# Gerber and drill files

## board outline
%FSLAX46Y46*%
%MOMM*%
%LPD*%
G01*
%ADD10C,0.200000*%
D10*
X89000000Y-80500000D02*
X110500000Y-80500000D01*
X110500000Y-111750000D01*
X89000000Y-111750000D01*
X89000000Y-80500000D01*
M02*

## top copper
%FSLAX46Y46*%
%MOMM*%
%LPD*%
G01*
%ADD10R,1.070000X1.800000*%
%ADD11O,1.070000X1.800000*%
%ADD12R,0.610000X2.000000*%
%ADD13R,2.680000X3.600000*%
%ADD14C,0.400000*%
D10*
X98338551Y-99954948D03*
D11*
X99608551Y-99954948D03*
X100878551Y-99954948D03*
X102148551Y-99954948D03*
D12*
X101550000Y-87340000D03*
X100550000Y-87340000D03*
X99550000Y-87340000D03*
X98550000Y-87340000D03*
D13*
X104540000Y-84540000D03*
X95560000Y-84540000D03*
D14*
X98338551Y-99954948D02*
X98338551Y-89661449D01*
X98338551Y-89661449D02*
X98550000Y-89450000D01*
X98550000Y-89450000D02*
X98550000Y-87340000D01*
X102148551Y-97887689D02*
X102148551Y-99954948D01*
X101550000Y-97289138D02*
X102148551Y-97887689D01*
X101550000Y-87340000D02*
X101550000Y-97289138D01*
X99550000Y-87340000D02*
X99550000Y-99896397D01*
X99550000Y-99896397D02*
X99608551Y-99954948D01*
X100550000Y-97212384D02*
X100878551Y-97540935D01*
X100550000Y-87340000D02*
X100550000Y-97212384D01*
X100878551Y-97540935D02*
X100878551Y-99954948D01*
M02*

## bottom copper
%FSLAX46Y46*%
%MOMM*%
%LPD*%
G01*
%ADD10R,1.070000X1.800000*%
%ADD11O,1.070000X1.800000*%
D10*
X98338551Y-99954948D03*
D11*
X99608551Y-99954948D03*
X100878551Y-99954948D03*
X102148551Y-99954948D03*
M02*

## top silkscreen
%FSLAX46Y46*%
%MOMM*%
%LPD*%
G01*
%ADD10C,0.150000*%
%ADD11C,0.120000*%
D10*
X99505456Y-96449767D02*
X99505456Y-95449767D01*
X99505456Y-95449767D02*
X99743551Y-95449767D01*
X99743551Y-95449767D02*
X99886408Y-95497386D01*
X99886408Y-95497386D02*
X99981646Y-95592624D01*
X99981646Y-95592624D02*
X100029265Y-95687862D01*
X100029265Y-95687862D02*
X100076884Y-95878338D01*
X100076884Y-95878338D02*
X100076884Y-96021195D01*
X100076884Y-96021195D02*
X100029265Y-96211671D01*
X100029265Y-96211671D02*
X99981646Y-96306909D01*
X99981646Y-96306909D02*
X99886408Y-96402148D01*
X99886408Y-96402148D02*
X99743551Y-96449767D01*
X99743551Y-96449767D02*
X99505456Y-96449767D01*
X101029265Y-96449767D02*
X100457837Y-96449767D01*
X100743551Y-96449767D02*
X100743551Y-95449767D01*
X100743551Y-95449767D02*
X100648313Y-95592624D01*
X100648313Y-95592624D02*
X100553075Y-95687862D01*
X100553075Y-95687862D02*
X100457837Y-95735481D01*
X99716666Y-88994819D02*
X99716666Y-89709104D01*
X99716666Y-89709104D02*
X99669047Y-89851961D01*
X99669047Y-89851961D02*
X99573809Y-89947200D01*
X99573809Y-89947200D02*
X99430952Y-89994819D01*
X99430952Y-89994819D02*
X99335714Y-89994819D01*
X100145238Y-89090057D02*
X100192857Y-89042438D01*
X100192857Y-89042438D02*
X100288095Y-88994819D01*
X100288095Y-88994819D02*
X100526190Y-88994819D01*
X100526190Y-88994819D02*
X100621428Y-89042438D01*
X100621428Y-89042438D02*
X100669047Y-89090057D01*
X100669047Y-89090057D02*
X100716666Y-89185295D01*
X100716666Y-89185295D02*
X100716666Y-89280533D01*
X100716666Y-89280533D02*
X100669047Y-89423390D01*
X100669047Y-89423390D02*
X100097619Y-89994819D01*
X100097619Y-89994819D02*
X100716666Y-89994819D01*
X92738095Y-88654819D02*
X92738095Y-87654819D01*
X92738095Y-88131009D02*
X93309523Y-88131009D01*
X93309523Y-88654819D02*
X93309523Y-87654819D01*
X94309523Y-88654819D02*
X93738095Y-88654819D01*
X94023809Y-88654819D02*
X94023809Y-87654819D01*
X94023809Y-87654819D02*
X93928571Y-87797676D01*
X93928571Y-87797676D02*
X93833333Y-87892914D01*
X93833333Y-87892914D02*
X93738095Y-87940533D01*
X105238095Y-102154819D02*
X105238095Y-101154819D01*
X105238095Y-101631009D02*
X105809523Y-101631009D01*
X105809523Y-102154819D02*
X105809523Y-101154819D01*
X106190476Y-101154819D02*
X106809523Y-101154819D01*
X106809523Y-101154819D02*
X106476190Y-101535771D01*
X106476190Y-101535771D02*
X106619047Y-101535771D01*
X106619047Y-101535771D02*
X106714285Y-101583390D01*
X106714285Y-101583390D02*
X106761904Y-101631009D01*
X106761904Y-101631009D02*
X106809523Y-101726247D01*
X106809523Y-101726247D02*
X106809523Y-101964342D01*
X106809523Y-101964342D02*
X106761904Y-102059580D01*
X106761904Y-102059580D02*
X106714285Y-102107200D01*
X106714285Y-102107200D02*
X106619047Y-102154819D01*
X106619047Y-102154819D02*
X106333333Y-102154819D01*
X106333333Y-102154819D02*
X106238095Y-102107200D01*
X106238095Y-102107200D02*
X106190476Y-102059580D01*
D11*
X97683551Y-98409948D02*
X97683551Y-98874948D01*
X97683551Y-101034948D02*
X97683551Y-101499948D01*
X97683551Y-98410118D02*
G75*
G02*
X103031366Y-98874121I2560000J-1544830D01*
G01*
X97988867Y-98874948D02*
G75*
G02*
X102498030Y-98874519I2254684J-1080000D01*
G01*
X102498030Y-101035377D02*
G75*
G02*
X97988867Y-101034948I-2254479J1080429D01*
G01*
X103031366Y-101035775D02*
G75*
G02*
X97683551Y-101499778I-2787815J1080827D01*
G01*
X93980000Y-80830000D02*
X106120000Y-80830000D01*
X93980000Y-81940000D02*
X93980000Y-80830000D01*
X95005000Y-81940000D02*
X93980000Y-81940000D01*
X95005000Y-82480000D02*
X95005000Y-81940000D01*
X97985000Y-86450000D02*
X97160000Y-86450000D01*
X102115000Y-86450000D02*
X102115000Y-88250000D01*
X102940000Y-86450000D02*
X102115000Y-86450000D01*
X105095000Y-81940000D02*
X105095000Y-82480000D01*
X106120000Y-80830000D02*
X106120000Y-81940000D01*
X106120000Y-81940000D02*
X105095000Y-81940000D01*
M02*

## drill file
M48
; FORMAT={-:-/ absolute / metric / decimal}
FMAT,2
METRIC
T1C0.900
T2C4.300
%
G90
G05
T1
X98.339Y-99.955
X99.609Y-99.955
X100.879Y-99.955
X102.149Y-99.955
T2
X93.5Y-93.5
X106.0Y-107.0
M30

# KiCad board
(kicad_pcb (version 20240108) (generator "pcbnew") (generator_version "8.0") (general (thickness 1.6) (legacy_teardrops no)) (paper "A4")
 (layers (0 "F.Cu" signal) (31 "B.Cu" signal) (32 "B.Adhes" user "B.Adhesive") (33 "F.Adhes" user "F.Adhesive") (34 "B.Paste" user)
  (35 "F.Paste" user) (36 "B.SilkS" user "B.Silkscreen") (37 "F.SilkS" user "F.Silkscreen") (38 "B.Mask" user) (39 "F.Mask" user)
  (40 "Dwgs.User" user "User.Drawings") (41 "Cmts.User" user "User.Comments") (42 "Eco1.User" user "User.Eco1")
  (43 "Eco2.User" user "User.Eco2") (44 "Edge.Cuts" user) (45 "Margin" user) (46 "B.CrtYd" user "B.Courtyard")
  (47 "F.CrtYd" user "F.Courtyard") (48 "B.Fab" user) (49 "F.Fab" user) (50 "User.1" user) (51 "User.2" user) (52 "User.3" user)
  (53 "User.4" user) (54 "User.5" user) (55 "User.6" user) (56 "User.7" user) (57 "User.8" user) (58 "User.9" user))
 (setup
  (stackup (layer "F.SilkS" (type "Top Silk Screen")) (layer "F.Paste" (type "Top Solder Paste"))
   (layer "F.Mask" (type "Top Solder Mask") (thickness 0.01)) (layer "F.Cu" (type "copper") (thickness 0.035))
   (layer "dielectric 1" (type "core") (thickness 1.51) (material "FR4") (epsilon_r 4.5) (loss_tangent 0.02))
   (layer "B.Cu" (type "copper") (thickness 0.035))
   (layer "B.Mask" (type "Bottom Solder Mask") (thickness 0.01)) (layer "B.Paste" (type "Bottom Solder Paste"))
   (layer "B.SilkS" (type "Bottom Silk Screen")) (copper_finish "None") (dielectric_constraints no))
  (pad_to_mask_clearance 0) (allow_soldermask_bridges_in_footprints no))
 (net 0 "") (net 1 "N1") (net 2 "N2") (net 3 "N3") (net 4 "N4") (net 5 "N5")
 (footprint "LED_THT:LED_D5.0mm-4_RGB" (layer "F.Cu") (at 98.338551 99.954948)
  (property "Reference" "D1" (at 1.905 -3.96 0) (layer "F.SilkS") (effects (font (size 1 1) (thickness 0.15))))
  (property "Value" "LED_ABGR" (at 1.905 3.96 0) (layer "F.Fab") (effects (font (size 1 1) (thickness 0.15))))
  (fp_line (start -0.655 -1.545) (end -0.655 -1.08) (stroke (width 0.12) (type solid)) (layer "F.SilkS"))
  (fp_line (start -0.655 1.08) (end -0.655 1.545) (stroke (width 0.12) (type solid)) (layer "F.SilkS"))
  (fp_arc (start -0.655 -1.54483) (mid 2.163456 -2.978809) (end 4.692815 -1.080827) (stroke (width 0.12) (type solid)) (layer "F.SilkS"))
  (fp_arc (start -0.349684 -1.08) (mid 1.904762 -2.5) (end 4.159479 -1.080429) (stroke (width 0.12) (type solid)) (layer "F.SilkS"))
  (fp_arc (start 4.159479 1.080429) (mid 1.904762 2.5) (end -0.349684 1.08) (stroke (width 0.12) (type solid)) (layer "F.SilkS"))
  (fp_arc (start 4.692815 1.080827) (mid 2.163456 2.978808) (end -0.655 1.54483) (stroke (width 0.12) (type solid)) (layer "F.SilkS"))
  (pad "1" thru_hole rect (at 0 0) (size 1.07 1.8) (drill 0.9) (layers "*.Cu" "*.Mask") (remove_unused_layers no) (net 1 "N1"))
  (pad "2" thru_hole oval (at 1.27 0) (size 1.07 1.8) (drill 0.9) (layers "*.Cu" "*.Mask") (remove_unused_layers no) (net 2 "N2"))
  (pad "3" thru_hole oval (at 2.54 0) (size 1.07 1.8) (drill 0.9) (layers "*.Cu" "*.Mask") (remove_unused_layers no) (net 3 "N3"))
  (pad "4" thru_hole oval (at 3.81 0) (size 1.07 1.8) (drill 0.9) (layers "*.Cu" "*.Mask") (remove_unused_layers no) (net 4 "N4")))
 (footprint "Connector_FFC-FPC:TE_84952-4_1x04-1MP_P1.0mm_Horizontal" (layer "F.Cu") (at 100.05 85.54 180)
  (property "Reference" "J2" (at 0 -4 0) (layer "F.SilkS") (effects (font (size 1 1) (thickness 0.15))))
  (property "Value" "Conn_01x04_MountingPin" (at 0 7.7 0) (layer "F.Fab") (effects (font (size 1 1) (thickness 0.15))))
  (fp_line (start 6.07 4.71) (end -6.07 4.71) (stroke (width 0.12) (type solid)) (layer "F.SilkS"))
  (fp_line (start 6.07 3.6) (end 6.07 4.71) (stroke (width 0.12) (type solid)) (layer "F.SilkS"))
  (fp_line (start 5.045 3.6) (end 6.07 3.6) (stroke (width 0.12) (type solid)) (layer "F.SilkS"))
  (fp_line (start 5.045 3.06) (end 5.045 3.6) (stroke (width 0.12) (type solid)) (layer "F.SilkS"))
  (fp_line (start 2.065 -0.91) (end 2.89 -0.91) (stroke (width 0.12) (type solid)) (layer "F.SilkS"))
  (fp_line (start -2.065 -0.91) (end -2.065 -2.71) (stroke (width 0.12) (type solid)) (layer "F.SilkS"))
  (fp_line (start -2.89 -0.91) (end -2.065 -0.91) (stroke (width 0.12) (type solid)) (layer "F.SilkS"))
  (fp_line (start -5.045 3.6) (end -5.045 3.06) (stroke (width 0.12) (type solid)) (layer "F.SilkS"))
  (fp_line (start -6.07 4.71) (end -6.07 3.6) (stroke (width 0.12) (type solid)) (layer "F.SilkS"))
  (fp_line (start -6.07 3.6) (end -5.045 3.6) (stroke (width 0.12) (type solid)) (layer "F.SilkS"))
  (pad "1" smd rect (at -1.5 -1.8 180) (size 0.61 2) (layers "F.Cu" "F.Paste" "F.Mask") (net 4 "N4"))
  (pad "2" smd rect (at -0.5 -1.8 180) (size 0.61 2) (layers "F.Cu" "F.Paste" "F.Mask") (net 3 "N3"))
  (pad "3" smd rect (at 0.5 -1.8 180) (size 0.61 2) (layers "F.Cu" "F.Paste" "F.Mask") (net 2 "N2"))
  (pad "4" smd rect (at 1.5 -1.8 180) (size 0.61 2) (layers "F.Cu" "F.Paste" "F.Mask") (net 1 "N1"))
  (pad "MP" smd rect (at -4.49 1 180) (size 2.68 3.6) (layers "F.Cu" "F.Paste" "F.Mask") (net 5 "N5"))
  (pad "MP" smd rect (at 4.49 1 180) (size 2.68 3.6) (layers "F.Cu" "F.Paste" "F.Mask") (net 5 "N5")))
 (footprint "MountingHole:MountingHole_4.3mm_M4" (layer "F.Cu") (at 93.5 93.5)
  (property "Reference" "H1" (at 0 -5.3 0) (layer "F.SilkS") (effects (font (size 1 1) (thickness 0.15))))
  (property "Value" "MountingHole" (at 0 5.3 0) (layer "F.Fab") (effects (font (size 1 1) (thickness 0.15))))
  (pad "" np_thru_hole circle (at 0 0) (size 4.3 4.3) (drill 4.3) (layers "*.Cu" "*.Mask")))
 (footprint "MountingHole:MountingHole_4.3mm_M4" (layer "F.Cu") (at 106 107)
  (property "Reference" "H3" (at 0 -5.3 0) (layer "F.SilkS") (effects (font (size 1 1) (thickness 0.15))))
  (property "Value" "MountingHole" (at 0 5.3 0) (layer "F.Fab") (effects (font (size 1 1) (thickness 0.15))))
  (pad "" np_thru_hole circle (at 0 0) (size 4.3 4.3) (drill 4.3) (layers "*.Cu" "*.Mask")))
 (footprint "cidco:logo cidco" (layer "B.Cu") (at 101 89.5 -90)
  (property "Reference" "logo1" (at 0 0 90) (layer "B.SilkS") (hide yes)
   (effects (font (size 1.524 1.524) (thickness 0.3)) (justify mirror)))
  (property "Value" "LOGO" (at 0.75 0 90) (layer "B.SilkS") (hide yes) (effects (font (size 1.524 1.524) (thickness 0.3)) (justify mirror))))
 (gr_rect (start 89 80.5) (end 110.5 111.75) (stroke (width 0.2) (type default)) (fill none) (layer "Edge.Cuts"))
 (segment (start 98.338551 99.954948) (end 98.338551 89.661449) (width 0.4) (layer "F.Cu") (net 1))
 (segment (start 98.338551 89.661449) (end 98.55 89.45) (width 0.4) (layer "F.Cu") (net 1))
 (segment (start 98.55 89.45) (end 98.55 87.34) (width 0.4) (layer "F.Cu") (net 1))
 (segment (start 102.148551 97.887689) (end 102.148551 99.954948) (width 0.4) (layer "F.Cu") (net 4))
 (segment (start 101.55 97.289138) (end 102.148551 97.887689) (width 0.4) (layer "F.Cu") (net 4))
 (segment (start 101.55 87.34) (end 101.55 97.289138) (width 0.4) (layer "F.Cu") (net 4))
 (segment (start 99.55 87.34) (end 99.55 99.896397) (width 0.4) (layer "F.Cu") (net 2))
 (segment (start 99.55 99.896397) (end 99.608551 99.954948) (width 0.4) (layer "F.Cu") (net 2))
 (segment (start 100.55 97.212384) (end 100.878551 97.540935) (width 0.4) (layer "F.Cu") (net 3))
 (segment (start 100.55 87.34) (end 100.55 97.212384) (width 0.4) (layer "F.Cu") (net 3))
 (segment (start 100.878551 97.540935) (end 100.878551 99.954948) (width 0.4) (layer "F.Cu") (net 3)))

